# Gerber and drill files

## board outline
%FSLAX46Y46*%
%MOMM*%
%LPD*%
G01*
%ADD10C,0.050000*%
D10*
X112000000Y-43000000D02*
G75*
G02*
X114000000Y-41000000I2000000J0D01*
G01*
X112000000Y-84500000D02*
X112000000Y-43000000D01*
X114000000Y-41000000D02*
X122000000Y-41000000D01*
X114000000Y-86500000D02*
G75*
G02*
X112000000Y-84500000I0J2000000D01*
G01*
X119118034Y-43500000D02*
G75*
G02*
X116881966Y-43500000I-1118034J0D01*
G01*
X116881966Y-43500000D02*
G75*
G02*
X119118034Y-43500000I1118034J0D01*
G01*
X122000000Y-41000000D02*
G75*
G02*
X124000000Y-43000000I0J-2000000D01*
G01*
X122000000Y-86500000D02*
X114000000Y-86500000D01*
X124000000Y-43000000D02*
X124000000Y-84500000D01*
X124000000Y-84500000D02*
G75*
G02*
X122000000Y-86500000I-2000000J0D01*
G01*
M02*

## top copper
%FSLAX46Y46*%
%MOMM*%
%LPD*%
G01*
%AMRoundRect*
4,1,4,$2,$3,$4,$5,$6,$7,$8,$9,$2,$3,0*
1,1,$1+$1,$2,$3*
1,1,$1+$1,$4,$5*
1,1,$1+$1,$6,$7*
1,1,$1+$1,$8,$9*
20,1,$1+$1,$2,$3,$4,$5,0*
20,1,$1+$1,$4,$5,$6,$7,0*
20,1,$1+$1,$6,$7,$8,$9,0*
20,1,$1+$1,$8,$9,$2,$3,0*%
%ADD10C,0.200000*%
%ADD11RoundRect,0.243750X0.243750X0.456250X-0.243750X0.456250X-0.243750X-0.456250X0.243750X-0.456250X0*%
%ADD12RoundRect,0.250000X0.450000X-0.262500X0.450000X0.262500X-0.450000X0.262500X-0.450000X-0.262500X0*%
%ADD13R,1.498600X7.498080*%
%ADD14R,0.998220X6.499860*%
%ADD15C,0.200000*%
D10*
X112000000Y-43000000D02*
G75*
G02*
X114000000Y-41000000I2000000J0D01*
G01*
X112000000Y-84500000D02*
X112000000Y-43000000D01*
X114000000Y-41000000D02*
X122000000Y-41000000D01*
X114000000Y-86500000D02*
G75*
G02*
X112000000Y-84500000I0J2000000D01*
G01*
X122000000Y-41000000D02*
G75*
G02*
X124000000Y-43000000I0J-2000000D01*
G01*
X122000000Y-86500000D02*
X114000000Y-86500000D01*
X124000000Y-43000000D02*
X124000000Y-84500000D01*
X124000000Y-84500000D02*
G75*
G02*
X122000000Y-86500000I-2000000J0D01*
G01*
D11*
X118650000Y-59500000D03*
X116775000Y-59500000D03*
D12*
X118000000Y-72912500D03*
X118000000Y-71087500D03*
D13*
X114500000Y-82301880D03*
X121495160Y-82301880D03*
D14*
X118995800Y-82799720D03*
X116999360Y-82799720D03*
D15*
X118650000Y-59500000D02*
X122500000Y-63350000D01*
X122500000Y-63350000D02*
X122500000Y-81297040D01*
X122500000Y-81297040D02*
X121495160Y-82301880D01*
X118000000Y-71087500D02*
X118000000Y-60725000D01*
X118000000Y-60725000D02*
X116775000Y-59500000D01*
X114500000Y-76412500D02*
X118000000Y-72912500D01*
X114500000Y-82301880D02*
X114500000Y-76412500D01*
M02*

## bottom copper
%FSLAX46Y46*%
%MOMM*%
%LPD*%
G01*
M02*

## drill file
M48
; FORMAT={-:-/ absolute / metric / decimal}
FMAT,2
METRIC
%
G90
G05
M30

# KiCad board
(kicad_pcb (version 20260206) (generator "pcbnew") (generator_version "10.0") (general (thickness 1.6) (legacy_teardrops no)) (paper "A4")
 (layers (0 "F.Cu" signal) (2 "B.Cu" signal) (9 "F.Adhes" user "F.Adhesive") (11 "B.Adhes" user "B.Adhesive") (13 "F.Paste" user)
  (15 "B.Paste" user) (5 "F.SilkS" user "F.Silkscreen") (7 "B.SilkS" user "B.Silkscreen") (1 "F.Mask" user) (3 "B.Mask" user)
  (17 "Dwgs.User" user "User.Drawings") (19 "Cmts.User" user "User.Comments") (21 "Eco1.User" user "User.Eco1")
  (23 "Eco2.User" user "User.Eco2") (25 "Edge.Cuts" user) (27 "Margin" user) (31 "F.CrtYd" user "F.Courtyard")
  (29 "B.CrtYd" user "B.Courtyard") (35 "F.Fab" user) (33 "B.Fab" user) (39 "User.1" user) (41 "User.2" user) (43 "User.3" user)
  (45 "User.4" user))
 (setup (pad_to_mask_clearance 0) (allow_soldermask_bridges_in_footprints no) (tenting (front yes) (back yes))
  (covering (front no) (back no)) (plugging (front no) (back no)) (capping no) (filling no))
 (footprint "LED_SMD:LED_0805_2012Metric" (layer "F.Cu") (at 117.7125 59.5 180)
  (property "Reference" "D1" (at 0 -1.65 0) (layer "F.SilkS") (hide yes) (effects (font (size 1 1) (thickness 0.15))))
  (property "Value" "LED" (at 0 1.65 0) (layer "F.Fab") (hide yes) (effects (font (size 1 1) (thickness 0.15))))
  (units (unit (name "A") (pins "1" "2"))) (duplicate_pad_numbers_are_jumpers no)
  (pad "1" smd roundrect (at -0.9375 0 180) (size 0.975 1.4) (layers "F.Cu" "F.Mask" "F.Paste") (roundrect_rratio 0.25) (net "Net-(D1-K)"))
  (pad "2" smd roundrect (at 0.9375 0 180) (size 0.975 1.4) (layers "F.Cu" "F.Mask" "F.Paste") (roundrect_rratio 0.25) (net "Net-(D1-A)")))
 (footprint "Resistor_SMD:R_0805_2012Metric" (layer "F.Cu") (at 118 72 90)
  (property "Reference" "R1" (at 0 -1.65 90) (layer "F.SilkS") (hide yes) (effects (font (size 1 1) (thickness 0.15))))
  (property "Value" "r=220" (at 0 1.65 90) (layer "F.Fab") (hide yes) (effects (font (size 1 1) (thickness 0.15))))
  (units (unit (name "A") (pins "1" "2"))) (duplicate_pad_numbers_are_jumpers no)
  (pad "1" smd roundrect (at -0.9125 0 90) (size 1.025 1.4) (layers "F.Cu" "F.Mask" "F.Paste") (roundrect_rratio 0.243902)
   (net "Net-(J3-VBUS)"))
  (pad "2" smd roundrect (at 0.9125 0 90) (size 1.025 1.4) (layers "F.Cu" "F.Mask" "F.Paste") (roundrect_rratio 0.243902) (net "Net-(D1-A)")))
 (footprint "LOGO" (layer "F.Cu") (at 113.5 46)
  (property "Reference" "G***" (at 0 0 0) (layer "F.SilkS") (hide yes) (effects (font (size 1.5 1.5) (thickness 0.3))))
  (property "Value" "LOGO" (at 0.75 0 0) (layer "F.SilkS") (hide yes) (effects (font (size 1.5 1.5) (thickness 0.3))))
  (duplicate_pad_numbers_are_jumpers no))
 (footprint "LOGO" (layer "F.Cu") (at 117.5 59.8175)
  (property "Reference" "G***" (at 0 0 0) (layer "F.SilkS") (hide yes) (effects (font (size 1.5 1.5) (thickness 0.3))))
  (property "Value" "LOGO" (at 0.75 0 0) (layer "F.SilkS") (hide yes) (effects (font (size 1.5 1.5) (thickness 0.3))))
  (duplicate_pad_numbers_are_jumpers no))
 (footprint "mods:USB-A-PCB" (layer "F.Cu") (at 117.99758 82.5 -90)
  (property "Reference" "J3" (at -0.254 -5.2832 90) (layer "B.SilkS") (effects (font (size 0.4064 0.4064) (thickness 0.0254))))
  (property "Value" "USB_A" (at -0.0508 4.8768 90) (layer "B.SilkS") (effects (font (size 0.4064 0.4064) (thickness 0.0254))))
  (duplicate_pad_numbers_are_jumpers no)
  (pad "5V" smd rect (at -0.19812 3.49758 270) (size 7.49808 1.4986) (layers "F.Cu" "F.Mask" "F.Paste"))
  (pad "GND" smd rect (at -0.19812 -3.49758 270) (size 7.49808 1.4986) (layers "F.Cu" "F.Mask" "F.Paste"))
  (pad "USB_" smd rect (at 0.29972 -0.99822 270) (size 6.49986 0.99822) (layers "F.Cu" "F.Mask" "F.Paste"))
  (pad "USB_" smd rect (at 0.29972 0.99822 270) (size 6.49986 0.99822) (layers "F.Cu" "F.Mask" "F.Paste")))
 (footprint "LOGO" (layer "F.Cu") (at 122.5 53.5)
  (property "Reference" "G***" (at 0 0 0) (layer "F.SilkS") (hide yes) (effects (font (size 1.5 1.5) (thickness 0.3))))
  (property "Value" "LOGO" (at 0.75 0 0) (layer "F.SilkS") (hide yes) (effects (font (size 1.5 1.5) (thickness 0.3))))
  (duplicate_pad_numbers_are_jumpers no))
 (gr_arc (start 112 43) (mid 112.585786 41.585786) (end 114 41) (stroke (width 0.2) (type default)) (layer "F.Cu"))
 (gr_line (start 112 84.5) (end 112 43) (stroke (width 0.2) (type default)) (layer "F.Cu"))
 (gr_line (start 114 41) (end 122 41) (stroke (width 0.2) (type default)) (layer "F.Cu"))
 (gr_arc (start 114 86.5) (mid 112.585786 85.914214) (end 112 84.5) (stroke (width 0.2) (type default)) (layer "F.Cu"))
 (gr_arc (start 122 41) (mid 123.414214 41.585786) (end 124 43) (stroke (width 0.2) (type default)) (layer "F.Cu"))
 (gr_line (start 122 86.5) (end 114 86.5) (stroke (width 0.2) (type default)) (layer "F.Cu"))
 (gr_line (start 124 43) (end 124 84.5) (stroke (width 0.2) (type default)) (layer "F.Cu"))
 (gr_arc (start 124 84.5) (mid 123.414214 85.914214) (end 122 86.5) (stroke (width 0.2) (type default)) (layer "F.Cu"))
 (gr_arc (start 112 43) (mid 112.585786 41.585786) (end 114 41) (stroke (width 0.05) (type default)) (layer "Edge.Cuts"))
 (gr_line (start 112 84.5) (end 112 43) (stroke (width 0.05) (type default)) (layer "Edge.Cuts"))
 (gr_line (start 114 41) (end 122 41) (stroke (width 0.05) (type default)) (layer "Edge.Cuts"))
 (gr_arc (start 114 86.5) (mid 112.585786 85.914214) (end 112 84.5) (stroke (width 0.05) (type default)) (layer "Edge.Cuts"))
 (gr_circle (center 118 43.5) (end 118.5 44.5) (stroke (width 0.05) (type default)) (fill no) (layer "Edge.Cuts"))
 (gr_arc (start 122 41) (mid 123.414214 41.585786) (end 124 43) (stroke (width 0.05) (type default)) (layer "Edge.Cuts"))
 (gr_line (start 122 86.5) (end 114 86.5) (stroke (width 0.05) (type default)) (layer "Edge.Cuts"))
 (gr_line (start 124 43) (end 124 84.5) (stroke (width 0.05) (type default)) (layer "Edge.Cuts"))
 (gr_arc (start 124 84.5) (mid 123.414214 85.914214) (end 122 86.5) (stroke (width 0.05) (type default)) (layer "Edge.Cuts"))
 (segment (start 118.65 59.5) (end 122.5 63.35) (width 0.2) (layer "F.Cu") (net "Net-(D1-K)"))
 (segment (start 122.5 63.35) (end 122.5 81.29704) (width 0.2) (layer "F.Cu") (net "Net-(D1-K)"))
 (segment (start 122.5 81.29704) (end 121.49516 82.30188) (width 0.2) (layer "F.Cu") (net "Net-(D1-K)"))
 (segment (start 118 71.0875) (end 118 60.725) (width 0.2) (layer "F.Cu") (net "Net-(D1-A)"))
 (segment (start 118 60.725) (end 116.775 59.5) (width 0.2) (layer "F.Cu") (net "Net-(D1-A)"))
 (segment (start 114.5 76.4125) (end 118 72.9125) (width 0.2) (layer "F.Cu") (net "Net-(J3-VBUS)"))
 (segment (start 114.5 82.30188) (end 114.5 76.4125) (width 0.2) (layer "F.Cu") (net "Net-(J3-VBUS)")))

